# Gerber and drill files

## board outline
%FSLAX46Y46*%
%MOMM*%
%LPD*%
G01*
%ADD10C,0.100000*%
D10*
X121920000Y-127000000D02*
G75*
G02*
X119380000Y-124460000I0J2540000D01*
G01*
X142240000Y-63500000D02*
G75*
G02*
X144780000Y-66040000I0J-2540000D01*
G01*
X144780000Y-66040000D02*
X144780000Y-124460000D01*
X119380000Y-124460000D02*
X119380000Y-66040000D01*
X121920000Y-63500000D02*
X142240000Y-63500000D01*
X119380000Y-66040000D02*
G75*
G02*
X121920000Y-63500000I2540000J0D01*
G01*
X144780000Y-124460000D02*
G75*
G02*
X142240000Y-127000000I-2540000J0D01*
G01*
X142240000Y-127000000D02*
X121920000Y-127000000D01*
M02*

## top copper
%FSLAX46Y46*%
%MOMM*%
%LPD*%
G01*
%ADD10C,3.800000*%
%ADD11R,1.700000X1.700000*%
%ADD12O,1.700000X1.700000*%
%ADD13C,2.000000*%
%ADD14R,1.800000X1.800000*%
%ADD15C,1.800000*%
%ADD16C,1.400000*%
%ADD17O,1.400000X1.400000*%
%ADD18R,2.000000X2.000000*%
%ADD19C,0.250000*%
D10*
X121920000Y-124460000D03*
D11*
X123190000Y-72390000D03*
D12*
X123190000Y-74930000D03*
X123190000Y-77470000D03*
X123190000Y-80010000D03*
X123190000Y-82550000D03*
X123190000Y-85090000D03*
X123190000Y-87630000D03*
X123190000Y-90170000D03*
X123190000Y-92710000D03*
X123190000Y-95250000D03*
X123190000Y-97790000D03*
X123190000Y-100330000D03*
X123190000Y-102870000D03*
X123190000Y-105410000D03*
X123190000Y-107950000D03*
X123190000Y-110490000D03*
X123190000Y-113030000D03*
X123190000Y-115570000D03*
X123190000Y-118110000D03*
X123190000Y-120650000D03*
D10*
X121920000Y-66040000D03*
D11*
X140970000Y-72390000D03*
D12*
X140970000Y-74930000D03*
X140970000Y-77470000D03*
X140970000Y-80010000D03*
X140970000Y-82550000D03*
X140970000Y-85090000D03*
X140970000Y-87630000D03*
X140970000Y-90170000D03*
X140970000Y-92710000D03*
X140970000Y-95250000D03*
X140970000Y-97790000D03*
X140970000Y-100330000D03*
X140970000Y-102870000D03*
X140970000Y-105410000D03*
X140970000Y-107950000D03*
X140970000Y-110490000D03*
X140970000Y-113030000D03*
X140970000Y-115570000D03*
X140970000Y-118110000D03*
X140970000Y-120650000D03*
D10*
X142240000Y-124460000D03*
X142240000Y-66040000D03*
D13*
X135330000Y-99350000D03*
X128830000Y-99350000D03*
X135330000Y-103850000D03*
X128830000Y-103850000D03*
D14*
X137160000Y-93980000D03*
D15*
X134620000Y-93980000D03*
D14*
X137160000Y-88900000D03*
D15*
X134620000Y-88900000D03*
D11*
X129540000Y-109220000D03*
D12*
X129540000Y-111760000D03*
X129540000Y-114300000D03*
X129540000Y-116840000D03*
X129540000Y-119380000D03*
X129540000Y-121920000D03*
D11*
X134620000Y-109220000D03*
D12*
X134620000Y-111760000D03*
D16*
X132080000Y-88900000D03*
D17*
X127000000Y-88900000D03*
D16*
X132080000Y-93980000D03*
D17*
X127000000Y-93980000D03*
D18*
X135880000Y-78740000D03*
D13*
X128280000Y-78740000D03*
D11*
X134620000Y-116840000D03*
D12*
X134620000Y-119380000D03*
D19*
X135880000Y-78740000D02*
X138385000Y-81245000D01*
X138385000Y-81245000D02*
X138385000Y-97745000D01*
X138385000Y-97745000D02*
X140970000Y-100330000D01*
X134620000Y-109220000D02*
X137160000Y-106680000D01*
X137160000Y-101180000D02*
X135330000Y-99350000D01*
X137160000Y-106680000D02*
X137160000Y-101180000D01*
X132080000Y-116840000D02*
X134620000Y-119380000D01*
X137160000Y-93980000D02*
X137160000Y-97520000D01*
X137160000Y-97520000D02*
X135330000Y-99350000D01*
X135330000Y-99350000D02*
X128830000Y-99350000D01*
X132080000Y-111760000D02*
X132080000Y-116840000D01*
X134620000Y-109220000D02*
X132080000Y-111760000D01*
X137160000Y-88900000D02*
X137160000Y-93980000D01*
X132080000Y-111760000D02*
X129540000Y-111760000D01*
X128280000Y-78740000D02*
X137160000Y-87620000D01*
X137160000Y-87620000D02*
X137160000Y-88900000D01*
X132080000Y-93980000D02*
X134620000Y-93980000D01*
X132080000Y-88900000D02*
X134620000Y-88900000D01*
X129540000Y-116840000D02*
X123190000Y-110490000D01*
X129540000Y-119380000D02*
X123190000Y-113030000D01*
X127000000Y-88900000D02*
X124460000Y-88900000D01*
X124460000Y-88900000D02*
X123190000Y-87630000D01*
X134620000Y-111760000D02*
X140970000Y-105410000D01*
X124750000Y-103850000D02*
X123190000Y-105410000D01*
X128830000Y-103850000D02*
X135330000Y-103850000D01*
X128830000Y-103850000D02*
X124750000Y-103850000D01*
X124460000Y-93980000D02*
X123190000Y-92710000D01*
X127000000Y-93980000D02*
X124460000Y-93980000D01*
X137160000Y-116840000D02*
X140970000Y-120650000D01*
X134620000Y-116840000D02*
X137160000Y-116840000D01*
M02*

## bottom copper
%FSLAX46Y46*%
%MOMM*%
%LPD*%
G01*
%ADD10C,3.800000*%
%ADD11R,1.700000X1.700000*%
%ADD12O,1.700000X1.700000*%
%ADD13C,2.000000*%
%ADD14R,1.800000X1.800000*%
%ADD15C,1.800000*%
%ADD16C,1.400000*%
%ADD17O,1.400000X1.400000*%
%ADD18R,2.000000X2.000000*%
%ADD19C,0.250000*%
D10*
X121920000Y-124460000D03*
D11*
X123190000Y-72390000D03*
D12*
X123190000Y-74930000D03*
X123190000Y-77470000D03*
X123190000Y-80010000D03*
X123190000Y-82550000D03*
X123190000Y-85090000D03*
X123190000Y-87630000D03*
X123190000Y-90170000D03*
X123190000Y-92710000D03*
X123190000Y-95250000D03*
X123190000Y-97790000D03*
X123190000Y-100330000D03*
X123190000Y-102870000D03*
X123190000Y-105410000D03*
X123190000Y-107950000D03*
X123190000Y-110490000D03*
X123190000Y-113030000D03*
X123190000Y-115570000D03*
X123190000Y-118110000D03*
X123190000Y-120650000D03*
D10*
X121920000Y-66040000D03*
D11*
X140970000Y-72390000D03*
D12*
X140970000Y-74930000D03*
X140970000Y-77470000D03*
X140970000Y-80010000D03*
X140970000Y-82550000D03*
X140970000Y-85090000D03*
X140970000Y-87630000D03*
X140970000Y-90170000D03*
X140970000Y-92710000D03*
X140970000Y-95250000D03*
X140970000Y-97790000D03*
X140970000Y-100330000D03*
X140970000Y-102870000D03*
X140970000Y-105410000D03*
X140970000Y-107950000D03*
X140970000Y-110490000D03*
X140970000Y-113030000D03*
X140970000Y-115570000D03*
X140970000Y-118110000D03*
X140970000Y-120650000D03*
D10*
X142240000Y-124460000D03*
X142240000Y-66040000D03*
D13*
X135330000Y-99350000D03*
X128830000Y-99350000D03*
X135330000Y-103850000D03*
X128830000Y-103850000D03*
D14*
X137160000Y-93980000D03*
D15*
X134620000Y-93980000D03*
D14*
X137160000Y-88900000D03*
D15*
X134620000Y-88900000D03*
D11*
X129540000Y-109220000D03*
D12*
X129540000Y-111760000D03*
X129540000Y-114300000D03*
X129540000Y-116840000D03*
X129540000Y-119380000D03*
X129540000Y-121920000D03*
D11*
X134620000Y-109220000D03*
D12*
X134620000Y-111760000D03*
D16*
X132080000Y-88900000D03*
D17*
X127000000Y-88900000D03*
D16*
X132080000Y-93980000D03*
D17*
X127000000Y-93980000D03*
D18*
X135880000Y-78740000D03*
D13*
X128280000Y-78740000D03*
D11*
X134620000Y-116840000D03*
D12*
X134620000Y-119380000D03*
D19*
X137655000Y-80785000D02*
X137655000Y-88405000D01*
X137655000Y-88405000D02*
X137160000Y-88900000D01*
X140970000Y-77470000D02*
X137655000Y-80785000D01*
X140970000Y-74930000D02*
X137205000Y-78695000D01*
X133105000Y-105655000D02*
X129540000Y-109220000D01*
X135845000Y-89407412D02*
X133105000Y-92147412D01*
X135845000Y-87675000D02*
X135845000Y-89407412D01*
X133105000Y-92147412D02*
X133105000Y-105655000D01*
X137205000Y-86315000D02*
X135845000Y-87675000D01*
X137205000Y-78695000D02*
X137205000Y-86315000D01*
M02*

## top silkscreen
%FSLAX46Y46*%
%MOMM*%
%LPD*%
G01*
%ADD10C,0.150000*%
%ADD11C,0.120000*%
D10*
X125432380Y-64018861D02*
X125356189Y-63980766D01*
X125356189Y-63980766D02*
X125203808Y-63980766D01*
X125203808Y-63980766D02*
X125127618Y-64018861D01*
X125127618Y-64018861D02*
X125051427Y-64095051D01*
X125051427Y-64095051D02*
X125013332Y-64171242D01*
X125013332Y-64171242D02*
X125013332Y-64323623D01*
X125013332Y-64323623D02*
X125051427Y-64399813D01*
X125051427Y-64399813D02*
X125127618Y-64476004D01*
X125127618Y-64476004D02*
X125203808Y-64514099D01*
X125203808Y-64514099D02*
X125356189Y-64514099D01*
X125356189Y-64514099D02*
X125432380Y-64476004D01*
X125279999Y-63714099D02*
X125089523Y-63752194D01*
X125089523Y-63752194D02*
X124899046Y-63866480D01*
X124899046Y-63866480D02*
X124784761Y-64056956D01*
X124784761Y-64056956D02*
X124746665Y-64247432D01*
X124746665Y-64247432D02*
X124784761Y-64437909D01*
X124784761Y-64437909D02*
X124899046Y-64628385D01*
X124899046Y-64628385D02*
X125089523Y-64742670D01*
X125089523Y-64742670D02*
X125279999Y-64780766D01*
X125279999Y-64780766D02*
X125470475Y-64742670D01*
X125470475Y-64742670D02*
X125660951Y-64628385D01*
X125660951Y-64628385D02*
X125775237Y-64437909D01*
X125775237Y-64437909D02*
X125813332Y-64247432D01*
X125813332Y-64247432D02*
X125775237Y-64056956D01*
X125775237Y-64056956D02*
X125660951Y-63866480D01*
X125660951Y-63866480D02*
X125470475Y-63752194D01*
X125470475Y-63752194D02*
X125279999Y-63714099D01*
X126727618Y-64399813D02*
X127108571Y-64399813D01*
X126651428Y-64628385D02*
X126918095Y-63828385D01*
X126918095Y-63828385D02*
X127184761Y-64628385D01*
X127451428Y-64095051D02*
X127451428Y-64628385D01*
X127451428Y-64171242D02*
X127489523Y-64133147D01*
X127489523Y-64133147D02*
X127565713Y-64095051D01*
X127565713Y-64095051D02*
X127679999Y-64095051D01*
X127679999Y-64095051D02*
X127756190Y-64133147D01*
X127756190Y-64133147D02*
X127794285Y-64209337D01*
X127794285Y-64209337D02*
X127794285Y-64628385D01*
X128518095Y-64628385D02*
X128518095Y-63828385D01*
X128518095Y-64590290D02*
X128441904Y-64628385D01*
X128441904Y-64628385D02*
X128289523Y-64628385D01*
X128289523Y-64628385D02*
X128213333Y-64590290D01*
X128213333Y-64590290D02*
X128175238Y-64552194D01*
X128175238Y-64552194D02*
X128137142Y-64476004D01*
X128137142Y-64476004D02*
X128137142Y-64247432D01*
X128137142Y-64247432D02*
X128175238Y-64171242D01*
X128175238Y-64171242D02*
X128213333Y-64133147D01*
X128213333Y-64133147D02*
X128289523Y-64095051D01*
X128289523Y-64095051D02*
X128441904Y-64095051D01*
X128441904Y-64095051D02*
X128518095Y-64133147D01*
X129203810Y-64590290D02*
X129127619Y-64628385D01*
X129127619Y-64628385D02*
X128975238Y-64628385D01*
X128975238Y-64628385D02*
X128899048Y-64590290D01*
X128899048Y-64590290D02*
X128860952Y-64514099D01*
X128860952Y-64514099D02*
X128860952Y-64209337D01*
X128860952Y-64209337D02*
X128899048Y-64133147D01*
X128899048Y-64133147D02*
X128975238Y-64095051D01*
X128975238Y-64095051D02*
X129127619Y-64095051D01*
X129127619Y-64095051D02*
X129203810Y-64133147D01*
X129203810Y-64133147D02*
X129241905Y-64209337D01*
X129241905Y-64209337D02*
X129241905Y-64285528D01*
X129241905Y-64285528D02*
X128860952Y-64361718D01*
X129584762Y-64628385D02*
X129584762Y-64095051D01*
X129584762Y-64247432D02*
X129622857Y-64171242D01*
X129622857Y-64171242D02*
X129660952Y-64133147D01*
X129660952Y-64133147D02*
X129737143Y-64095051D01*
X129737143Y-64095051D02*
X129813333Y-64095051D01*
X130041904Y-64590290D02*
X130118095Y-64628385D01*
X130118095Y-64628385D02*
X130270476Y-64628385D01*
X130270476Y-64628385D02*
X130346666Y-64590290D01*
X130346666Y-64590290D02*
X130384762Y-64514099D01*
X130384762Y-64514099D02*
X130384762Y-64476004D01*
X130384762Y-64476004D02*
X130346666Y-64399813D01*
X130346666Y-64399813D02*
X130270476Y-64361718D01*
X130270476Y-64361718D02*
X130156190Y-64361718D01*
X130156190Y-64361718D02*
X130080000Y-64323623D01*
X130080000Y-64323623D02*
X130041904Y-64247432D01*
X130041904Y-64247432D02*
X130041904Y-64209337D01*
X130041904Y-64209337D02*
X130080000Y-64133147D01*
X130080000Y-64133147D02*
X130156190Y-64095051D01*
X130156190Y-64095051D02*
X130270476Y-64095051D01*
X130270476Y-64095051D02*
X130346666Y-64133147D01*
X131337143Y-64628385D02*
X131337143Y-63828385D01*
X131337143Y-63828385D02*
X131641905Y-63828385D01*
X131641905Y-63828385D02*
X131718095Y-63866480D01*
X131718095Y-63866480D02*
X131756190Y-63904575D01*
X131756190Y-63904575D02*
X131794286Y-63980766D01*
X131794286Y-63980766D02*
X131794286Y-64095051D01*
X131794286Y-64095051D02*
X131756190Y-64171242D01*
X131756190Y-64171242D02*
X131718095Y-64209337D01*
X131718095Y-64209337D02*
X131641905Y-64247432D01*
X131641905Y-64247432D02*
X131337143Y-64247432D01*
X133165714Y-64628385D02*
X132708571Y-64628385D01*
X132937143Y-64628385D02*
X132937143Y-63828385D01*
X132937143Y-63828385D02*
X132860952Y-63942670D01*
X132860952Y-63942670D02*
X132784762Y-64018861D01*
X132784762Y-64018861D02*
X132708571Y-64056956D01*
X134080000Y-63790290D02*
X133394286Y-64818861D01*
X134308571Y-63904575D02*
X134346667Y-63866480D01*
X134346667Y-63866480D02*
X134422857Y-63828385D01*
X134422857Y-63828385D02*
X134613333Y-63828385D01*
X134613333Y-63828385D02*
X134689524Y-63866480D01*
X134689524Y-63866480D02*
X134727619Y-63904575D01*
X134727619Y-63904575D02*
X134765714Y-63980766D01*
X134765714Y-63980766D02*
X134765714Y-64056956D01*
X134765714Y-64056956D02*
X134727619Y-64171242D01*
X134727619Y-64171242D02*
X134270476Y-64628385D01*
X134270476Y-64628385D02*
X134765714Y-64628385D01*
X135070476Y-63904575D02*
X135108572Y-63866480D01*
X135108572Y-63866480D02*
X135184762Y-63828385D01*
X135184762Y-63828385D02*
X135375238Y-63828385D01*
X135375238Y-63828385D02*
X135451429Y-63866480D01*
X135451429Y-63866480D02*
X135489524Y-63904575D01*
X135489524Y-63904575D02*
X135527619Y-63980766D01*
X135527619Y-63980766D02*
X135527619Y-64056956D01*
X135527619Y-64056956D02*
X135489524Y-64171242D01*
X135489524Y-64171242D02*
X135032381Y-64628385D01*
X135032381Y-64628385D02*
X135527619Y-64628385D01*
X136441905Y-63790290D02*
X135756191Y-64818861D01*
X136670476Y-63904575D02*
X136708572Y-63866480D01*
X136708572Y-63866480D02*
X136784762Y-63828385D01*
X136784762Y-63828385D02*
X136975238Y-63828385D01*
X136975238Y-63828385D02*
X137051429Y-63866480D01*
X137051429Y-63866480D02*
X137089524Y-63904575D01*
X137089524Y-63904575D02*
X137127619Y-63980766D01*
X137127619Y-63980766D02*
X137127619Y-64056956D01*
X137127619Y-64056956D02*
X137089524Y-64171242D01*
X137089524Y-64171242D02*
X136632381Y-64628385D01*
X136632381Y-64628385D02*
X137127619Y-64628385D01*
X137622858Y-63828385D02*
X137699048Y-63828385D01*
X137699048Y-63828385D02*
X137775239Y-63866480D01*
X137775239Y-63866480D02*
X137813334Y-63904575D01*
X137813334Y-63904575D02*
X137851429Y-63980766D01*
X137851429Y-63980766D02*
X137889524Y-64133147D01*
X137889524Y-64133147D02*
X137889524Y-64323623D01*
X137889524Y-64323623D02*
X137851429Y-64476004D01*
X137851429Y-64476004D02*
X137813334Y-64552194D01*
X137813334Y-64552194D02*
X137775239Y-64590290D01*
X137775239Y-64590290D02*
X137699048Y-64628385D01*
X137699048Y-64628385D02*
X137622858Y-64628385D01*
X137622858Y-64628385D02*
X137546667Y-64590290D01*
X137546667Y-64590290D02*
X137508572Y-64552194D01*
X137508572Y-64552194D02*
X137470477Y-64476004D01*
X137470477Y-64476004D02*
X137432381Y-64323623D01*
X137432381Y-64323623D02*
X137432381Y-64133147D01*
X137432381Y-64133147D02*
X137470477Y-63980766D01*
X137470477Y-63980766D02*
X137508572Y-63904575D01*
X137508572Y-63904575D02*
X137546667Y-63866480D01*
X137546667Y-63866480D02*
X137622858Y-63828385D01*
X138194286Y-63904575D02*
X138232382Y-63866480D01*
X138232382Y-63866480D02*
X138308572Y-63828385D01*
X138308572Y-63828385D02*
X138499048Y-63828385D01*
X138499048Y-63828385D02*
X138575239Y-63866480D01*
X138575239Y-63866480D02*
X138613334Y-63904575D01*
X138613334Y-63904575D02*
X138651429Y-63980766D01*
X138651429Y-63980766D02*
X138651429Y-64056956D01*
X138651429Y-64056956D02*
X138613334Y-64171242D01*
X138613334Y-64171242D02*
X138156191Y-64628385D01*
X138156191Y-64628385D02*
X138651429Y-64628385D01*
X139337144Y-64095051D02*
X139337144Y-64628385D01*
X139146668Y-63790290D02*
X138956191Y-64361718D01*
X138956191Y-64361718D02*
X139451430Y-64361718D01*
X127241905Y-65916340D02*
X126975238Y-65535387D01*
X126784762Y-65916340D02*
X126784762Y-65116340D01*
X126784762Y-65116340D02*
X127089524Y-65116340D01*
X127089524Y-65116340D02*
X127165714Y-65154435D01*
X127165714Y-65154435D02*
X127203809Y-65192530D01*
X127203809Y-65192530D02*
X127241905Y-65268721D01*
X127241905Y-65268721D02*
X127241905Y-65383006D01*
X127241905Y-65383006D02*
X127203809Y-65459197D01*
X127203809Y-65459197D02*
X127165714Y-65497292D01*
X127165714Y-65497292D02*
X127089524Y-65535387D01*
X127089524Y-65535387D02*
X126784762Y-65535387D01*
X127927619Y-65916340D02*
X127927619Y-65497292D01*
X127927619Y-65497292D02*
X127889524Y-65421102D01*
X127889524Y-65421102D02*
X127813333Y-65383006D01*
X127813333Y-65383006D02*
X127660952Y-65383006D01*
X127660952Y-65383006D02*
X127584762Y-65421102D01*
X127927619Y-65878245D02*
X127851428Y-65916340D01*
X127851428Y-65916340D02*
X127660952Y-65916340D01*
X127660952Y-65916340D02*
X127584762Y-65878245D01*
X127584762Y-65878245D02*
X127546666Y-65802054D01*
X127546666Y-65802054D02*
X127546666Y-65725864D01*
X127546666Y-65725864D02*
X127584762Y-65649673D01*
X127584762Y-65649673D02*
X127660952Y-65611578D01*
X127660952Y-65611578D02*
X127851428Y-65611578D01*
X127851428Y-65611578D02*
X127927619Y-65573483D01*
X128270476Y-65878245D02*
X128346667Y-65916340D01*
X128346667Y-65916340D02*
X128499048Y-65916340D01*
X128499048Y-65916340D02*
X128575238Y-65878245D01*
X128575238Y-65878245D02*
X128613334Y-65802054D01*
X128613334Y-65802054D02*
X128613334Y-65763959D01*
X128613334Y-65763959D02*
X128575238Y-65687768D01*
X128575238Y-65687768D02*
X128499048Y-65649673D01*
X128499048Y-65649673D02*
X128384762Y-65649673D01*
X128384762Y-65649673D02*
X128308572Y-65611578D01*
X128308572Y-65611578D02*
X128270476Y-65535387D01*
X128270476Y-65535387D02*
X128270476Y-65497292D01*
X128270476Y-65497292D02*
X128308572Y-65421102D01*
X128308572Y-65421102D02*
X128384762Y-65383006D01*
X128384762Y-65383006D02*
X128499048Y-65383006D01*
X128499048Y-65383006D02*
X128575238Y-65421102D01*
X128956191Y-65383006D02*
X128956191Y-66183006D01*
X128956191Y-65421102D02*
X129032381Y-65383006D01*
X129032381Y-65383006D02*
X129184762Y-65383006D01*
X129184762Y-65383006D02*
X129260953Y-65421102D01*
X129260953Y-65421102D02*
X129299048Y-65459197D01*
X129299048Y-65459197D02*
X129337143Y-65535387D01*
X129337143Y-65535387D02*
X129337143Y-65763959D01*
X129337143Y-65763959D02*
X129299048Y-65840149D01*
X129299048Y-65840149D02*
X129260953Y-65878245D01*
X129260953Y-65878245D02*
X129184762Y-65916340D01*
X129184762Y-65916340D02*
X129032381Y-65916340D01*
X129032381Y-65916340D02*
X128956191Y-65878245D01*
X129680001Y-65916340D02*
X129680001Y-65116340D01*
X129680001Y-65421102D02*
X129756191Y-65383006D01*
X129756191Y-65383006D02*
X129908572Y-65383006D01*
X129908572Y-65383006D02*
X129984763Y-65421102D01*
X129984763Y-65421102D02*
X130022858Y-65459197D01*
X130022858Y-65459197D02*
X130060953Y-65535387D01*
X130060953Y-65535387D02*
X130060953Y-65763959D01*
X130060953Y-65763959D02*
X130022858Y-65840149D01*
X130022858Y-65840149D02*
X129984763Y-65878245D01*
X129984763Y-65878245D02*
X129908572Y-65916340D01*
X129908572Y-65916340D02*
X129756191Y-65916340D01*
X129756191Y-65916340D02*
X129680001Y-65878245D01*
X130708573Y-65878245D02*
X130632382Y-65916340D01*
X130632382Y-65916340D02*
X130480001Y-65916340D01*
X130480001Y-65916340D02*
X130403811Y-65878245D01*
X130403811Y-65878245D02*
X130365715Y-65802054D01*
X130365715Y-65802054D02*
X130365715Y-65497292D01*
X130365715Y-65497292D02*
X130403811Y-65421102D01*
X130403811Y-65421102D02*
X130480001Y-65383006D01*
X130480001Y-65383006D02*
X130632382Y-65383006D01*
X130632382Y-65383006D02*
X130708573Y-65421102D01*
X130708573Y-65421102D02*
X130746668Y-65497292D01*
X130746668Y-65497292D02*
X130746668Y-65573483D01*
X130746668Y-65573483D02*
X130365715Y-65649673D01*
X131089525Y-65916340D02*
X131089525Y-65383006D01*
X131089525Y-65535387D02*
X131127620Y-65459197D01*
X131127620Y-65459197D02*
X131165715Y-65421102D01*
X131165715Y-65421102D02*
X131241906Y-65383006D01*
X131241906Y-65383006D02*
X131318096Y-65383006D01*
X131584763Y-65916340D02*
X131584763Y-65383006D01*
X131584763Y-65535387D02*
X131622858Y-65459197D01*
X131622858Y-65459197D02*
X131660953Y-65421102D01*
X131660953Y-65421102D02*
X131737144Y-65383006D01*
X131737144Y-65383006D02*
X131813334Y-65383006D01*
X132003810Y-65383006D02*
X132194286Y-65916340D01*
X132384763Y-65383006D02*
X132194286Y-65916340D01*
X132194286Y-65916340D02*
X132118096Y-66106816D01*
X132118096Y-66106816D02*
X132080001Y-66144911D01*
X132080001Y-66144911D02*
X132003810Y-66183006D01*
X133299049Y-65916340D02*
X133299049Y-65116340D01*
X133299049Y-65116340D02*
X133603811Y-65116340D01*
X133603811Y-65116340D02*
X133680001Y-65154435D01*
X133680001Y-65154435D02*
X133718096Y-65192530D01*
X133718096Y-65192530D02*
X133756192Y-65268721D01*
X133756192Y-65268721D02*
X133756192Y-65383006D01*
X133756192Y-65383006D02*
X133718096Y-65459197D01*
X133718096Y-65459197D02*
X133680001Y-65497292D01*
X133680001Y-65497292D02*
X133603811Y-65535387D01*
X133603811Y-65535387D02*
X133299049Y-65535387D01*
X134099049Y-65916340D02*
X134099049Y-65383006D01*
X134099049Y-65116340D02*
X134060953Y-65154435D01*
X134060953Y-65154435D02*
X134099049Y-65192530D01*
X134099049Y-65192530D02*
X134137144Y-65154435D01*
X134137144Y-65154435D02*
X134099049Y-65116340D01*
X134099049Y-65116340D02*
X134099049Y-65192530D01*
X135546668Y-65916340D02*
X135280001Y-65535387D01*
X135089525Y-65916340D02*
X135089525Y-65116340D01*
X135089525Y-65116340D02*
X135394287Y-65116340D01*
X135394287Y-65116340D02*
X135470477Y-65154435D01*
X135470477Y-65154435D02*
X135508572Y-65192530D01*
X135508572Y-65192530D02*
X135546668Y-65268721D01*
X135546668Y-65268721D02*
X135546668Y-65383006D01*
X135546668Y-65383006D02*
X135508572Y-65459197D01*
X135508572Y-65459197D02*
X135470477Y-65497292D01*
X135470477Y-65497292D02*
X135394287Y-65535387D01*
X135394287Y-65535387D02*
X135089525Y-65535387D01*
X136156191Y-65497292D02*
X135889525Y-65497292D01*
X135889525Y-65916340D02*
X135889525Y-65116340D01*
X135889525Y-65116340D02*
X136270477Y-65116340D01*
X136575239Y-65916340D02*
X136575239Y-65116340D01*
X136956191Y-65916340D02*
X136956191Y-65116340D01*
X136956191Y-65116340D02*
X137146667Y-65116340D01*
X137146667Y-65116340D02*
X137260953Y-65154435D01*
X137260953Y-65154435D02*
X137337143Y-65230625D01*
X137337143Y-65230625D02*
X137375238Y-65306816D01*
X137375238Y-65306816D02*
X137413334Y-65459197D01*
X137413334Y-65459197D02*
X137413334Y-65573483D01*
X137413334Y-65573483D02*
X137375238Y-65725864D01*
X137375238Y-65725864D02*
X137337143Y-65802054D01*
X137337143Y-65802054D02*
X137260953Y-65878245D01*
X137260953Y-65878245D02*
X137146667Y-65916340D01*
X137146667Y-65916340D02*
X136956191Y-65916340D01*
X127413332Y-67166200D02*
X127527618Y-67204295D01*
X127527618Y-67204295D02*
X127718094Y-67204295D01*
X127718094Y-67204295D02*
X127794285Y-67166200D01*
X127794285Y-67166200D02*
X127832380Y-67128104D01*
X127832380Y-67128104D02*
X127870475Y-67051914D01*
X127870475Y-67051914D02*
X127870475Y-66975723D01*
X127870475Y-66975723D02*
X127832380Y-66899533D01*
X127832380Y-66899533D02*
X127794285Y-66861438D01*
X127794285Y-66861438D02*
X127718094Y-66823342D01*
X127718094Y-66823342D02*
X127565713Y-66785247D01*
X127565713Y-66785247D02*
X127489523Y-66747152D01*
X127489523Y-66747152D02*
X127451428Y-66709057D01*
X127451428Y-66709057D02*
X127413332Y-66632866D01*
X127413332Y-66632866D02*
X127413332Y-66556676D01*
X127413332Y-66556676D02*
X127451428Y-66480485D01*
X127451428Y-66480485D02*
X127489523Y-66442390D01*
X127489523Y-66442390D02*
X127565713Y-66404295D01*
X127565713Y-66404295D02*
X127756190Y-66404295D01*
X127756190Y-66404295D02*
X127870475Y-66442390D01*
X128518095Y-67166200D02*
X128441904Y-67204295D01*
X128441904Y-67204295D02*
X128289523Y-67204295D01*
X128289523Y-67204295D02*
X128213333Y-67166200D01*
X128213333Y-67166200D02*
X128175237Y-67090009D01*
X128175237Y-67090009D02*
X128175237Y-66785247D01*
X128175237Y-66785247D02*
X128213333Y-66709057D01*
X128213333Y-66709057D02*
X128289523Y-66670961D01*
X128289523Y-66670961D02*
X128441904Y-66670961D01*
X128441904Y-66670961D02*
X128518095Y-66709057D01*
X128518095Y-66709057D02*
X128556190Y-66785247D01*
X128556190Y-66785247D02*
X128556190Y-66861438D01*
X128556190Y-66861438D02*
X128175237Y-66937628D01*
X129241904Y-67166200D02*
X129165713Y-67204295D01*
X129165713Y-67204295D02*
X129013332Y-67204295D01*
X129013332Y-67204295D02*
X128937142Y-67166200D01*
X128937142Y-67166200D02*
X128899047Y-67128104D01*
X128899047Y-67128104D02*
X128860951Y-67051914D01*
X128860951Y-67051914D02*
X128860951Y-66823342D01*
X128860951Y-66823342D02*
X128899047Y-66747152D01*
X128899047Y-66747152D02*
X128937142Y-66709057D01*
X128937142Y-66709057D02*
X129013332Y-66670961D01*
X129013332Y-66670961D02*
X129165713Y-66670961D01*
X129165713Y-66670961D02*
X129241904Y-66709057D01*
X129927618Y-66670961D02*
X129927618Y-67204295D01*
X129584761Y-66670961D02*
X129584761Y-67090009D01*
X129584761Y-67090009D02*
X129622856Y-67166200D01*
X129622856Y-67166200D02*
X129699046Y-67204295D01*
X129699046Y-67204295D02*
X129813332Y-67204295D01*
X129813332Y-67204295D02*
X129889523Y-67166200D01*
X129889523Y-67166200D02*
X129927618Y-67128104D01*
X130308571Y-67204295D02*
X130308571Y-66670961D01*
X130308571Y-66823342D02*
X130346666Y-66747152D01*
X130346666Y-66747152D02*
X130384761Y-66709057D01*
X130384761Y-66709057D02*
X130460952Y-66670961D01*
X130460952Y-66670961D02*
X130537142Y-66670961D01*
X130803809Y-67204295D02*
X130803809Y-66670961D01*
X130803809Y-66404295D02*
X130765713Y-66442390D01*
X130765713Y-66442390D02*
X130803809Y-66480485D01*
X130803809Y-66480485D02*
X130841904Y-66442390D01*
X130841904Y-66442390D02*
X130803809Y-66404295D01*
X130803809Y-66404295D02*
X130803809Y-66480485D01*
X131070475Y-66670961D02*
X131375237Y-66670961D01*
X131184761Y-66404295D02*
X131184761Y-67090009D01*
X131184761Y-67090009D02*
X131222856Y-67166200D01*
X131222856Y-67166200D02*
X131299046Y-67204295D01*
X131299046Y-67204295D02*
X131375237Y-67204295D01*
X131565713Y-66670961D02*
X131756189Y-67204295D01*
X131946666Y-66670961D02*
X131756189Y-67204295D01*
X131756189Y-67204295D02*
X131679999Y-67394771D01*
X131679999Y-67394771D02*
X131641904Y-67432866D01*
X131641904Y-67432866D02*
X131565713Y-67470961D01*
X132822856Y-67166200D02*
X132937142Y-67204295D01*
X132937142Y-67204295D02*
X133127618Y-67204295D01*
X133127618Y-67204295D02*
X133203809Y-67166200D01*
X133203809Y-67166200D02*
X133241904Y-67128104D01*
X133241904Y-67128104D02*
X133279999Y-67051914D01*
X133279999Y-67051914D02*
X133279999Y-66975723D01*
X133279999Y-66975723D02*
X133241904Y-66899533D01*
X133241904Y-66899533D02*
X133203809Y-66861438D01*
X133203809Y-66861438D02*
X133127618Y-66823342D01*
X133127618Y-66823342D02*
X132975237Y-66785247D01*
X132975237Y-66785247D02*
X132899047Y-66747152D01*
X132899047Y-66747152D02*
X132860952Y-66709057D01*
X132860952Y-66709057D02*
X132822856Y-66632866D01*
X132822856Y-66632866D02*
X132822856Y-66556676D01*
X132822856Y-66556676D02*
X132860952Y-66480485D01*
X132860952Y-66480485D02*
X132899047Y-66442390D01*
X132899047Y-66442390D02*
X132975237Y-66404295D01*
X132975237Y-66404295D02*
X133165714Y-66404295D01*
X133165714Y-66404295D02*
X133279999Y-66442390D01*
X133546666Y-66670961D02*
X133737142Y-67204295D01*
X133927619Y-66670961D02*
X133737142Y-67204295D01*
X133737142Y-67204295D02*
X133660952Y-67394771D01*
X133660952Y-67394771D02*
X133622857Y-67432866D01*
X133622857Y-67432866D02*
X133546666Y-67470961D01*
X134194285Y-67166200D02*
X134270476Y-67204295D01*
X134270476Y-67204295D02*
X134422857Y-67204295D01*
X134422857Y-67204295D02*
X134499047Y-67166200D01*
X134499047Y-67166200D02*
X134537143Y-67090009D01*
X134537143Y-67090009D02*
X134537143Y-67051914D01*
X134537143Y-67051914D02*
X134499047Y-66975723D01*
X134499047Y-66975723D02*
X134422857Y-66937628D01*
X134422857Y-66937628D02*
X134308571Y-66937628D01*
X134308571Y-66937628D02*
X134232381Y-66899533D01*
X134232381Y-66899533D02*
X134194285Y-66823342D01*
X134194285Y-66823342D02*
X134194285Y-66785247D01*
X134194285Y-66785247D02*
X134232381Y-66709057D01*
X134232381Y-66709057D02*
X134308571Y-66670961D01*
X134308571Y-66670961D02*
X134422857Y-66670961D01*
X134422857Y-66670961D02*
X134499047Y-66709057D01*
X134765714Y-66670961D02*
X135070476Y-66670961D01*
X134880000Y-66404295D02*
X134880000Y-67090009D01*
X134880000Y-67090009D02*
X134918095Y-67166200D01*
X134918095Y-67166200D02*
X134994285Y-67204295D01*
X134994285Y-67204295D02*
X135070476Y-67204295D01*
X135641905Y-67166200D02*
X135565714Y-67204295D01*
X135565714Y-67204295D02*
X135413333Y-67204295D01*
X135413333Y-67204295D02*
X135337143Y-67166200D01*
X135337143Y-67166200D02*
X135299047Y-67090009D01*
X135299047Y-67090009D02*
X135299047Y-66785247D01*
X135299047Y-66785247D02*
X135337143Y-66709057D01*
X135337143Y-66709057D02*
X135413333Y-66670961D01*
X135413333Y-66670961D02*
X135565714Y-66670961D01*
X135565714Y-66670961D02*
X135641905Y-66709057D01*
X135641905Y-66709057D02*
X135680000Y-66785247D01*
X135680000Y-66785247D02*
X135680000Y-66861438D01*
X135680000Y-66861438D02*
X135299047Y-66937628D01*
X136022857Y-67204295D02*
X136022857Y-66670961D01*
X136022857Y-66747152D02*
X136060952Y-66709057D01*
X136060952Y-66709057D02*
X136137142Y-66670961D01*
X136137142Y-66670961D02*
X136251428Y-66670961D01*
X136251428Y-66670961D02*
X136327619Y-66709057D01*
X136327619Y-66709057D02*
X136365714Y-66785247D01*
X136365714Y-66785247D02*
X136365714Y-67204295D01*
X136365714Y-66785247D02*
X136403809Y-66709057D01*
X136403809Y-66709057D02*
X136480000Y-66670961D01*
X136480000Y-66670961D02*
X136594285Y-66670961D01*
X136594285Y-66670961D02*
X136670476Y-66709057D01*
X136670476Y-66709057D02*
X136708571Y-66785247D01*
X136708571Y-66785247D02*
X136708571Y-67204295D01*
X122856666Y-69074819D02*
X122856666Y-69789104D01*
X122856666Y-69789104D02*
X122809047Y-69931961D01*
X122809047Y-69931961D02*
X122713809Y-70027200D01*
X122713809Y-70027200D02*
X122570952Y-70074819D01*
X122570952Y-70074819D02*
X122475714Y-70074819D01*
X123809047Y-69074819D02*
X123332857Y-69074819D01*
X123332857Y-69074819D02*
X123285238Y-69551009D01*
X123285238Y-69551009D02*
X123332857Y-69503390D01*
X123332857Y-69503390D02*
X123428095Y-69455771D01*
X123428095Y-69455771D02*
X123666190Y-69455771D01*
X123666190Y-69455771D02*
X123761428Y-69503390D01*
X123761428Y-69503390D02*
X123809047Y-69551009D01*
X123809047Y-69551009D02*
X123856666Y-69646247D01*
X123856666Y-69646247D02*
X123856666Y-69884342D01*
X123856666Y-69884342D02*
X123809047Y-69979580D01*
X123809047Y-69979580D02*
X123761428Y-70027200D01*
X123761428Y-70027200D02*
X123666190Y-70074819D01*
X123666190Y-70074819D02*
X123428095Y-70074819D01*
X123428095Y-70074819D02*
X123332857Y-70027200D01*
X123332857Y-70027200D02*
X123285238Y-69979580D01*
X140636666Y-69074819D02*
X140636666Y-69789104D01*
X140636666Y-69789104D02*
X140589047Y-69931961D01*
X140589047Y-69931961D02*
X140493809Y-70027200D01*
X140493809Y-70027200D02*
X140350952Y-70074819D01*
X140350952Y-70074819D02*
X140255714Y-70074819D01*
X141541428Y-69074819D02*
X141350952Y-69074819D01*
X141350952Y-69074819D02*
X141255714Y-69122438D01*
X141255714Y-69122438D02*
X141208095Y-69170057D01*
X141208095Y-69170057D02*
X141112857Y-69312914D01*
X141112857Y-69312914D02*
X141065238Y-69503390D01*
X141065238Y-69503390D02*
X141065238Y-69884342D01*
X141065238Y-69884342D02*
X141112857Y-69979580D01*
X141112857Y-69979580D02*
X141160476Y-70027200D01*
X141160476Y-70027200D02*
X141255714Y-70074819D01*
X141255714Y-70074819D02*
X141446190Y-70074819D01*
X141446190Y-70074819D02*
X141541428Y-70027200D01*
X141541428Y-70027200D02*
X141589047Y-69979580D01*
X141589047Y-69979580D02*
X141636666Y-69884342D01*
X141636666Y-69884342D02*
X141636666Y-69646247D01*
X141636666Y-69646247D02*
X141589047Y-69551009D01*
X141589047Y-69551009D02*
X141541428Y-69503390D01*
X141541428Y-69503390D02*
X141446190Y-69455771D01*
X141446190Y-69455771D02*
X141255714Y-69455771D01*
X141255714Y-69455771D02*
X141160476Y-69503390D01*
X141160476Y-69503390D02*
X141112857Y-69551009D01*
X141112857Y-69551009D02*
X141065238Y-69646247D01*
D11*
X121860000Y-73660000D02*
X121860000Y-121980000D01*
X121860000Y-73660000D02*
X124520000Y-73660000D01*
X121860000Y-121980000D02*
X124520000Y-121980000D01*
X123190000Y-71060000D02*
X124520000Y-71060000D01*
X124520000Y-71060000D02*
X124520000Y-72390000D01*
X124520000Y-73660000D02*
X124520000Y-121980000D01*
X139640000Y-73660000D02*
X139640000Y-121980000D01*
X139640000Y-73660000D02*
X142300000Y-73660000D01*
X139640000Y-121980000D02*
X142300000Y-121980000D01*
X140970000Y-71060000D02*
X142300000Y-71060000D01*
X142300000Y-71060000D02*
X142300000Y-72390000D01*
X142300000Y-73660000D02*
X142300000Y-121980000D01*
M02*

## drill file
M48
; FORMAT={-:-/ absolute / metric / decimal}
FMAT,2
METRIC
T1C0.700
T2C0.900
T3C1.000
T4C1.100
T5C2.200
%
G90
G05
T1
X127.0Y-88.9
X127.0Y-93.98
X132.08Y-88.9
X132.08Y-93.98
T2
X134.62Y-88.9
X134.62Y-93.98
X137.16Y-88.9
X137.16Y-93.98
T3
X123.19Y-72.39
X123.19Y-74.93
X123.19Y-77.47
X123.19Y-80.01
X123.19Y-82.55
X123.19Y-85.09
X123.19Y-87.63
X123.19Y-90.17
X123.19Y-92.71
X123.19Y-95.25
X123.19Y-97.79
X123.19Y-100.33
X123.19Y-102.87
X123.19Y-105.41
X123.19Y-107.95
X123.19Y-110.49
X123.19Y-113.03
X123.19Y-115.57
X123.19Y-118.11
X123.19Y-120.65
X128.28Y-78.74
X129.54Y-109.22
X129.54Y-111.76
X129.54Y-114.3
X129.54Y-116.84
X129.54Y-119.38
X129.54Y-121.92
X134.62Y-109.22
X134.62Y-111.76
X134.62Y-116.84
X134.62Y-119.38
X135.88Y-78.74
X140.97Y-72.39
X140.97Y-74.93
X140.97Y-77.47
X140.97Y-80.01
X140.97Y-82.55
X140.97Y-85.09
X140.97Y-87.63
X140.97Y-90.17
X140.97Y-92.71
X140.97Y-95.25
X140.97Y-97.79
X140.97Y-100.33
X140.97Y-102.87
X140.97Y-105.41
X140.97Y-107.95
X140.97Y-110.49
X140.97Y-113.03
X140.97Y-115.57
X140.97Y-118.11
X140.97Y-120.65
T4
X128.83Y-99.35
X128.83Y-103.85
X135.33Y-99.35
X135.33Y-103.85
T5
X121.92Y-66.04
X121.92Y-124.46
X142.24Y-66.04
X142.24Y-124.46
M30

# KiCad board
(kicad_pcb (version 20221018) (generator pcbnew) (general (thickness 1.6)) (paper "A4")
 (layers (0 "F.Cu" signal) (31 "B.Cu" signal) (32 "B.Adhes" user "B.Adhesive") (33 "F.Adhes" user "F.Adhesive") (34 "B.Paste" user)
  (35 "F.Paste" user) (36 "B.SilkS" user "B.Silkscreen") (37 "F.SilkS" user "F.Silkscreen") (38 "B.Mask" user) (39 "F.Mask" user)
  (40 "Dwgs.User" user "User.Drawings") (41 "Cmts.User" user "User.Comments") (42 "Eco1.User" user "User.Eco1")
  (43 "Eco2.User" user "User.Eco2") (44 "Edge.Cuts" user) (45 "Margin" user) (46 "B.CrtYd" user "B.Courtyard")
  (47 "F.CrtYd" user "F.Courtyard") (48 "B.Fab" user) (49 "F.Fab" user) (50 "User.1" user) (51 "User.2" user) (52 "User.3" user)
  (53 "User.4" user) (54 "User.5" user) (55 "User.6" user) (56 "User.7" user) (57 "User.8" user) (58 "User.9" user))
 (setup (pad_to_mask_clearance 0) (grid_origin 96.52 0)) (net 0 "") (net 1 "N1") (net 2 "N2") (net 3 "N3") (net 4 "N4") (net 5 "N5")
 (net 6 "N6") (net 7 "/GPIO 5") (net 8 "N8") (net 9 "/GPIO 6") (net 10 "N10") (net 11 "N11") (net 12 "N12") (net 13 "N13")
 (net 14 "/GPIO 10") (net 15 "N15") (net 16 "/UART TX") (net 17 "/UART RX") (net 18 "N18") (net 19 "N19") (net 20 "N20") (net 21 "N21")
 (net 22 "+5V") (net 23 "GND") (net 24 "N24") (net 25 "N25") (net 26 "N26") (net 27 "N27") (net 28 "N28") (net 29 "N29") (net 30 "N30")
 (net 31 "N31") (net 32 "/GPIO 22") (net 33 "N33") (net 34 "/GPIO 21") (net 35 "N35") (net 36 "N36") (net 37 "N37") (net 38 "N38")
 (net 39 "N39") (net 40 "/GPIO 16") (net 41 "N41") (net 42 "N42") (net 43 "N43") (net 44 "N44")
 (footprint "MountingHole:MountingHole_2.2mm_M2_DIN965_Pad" (layer "F.Cu") (at 121.92 124.46)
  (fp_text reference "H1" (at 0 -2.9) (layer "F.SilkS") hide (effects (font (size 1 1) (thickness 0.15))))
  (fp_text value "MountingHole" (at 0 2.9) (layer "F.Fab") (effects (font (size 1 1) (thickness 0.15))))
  (pad "1" thru_hole circle (at 0 0) (size 3.8 3.8) (drill 2.2) (layers "*.Cu" "*.Mask")))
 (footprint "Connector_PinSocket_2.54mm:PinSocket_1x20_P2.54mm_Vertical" (layer "F.Cu") (at 123.19 72.39)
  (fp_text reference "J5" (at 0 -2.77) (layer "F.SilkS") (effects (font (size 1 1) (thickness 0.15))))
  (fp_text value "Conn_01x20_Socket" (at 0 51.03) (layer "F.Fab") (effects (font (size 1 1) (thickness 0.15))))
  (fp_line (start -1.33 1.27) (end -1.33 49.59) (stroke (width 0.12) (type solid)) (layer "F.SilkS"))
  (fp_line (start -1.33 1.27) (end 1.33 1.27) (stroke (width 0.12) (type solid)) (layer "F.SilkS"))
  (fp_line (start -1.33 49.59) (end 1.33 49.59) (stroke (width 0.12) (type solid)) (layer "F.SilkS"))
  (fp_line (start 0 -1.33) (end 1.33 -1.33) (stroke (width 0.12) (type solid)) (layer "F.SilkS"))
  (fp_line (start 1.33 -1.33) (end 1.33 0) (stroke (width 0.12) (type solid)) (layer "F.SilkS"))
  (fp_line (start 1.33 1.27) (end 1.33 49.59) (stroke (width 0.12) (type solid)) (layer "F.SilkS"))
  (pad "1" thru_hole rect (at 0 0) (size 1.7 1.7) (drill 1) (layers "*.Cu" "*.Mask") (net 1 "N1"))
  (pad "2" thru_hole oval (at 0 2.54) (size 1.7 1.7) (drill 1) (layers "*.Cu" "*.Mask") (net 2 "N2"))
  (pad "3" thru_hole oval (at 0 5.08) (size 1.7 1.7) (drill 1) (layers "*.Cu" "*.Mask") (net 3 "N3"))
  (pad "4" thru_hole oval (at 0 7.62) (size 1.7 1.7) (drill 1) (layers "*.Cu" "*.Mask") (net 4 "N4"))
  (pad "5" thru_hole oval (at 0 10.16) (size 1.7 1.7) (drill 1) (layers "*.Cu" "*.Mask") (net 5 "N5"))
  (pad "6" thru_hole oval (at 0 12.7) (size 1.7 1.7) (drill 1) (layers "*.Cu" "*.Mask") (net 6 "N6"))
  (pad "7" thru_hole oval (at 0 15.24) (size 1.7 1.7) (drill 1) (layers "*.Cu" "*.Mask") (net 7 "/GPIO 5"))
  (pad "8" thru_hole oval (at 0 17.78) (size 1.7 1.7) (drill 1) (layers "*.Cu" "*.Mask") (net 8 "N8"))
  (pad "9" thru_hole oval (at 0 20.32) (size 1.7 1.7) (drill 1) (layers "*.Cu" "*.Mask") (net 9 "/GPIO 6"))
  (pad "10" thru_hole oval (at 0 22.86) (size 1.7 1.7) (drill 1) (layers "*.Cu" "*.Mask") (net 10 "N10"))
  (pad "11" thru_hole oval (at 0 25.4) (size 1.7 1.7) (drill 1) (layers "*.Cu" "*.Mask") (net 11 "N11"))
  (pad "12" thru_hole oval (at 0 27.94) (size 1.7 1.7) (drill 1) (layers "*.Cu" "*.Mask") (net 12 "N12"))
  (pad "13" thru_hole oval (at 0 30.48) (size 1.7 1.7) (drill 1) (layers "*.Cu" "*.Mask") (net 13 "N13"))
  (pad "14" thru_hole oval (at 0 33.02) (size 1.7 1.7) (drill 1) (layers "*.Cu" "*.Mask") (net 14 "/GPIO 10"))
  (pad "15" thru_hole oval (at 0 35.56) (size 1.7 1.7) (drill 1) (layers "*.Cu" "*.Mask") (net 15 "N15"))
  (pad "16" thru_hole oval (at 0 38.1) (size 1.7 1.7) (drill 1) (layers "*.Cu" "*.Mask") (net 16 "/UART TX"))
  (pad "17" thru_hole oval (at 0 40.64) (size 1.7 1.7) (drill 1) (layers "*.Cu" "*.Mask") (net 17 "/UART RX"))
  (pad "18" thru_hole oval (at 0 43.18) (size 1.7 1.7) (drill 1) (layers "*.Cu" "*.Mask") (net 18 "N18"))
  (pad "19" thru_hole oval (at 0 45.72) (size 1.7 1.7) (drill 1) (layers "*.Cu" "*.Mask") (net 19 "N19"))
  (pad "20" thru_hole oval (at 0 48.26) (size 1.7 1.7) (drill 1) (layers "*.Cu" "*.Mask") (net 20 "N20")))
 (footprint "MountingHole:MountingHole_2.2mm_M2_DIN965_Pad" (layer "F.Cu") (at 121.92 66.04)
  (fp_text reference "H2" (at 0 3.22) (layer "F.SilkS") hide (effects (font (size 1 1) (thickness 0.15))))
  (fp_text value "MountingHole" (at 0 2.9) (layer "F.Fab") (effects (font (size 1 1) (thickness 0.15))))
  (pad "1" thru_hole circle (at 0 0) (size 3.8 3.8) (drill 2.2) (layers "*.Cu" "*.Mask")))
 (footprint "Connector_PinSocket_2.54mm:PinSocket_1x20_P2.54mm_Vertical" (layer "F.Cu") (at 140.97 72.39)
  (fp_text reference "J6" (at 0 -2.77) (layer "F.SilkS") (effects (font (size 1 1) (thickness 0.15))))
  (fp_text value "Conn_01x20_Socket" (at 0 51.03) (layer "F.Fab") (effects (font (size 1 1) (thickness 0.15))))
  (fp_line (start -1.33 1.27) (end -1.33 49.59) (stroke (width 0.12) (type solid)) (layer "F.SilkS"))
  (fp_line (start -1.33 1.27) (end 1.33 1.27) (stroke (width 0.12) (type solid)) (layer "F.SilkS"))
  (fp_line (start -1.33 49.59) (end 1.33 49.59) (stroke (width 0.12) (type solid)) (layer "F.SilkS"))
  (fp_line (start 0 -1.33) (end 1.33 -1.33) (stroke (width 0.12) (type solid)) (layer "F.SilkS"))
  (fp_line (start 1.33 -1.33) (end 1.33 0) (stroke (width 0.12) (type solid)) (layer "F.SilkS"))
  (fp_line (start 1.33 1.27) (end 1.33 49.59) (stroke (width 0.12) (type solid)) (layer "F.SilkS"))
  (pad "1" thru_hole rect (at 0 0) (size 1.7 1.7) (drill 1) (layers "*.Cu" "*.Mask") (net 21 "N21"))
  (pad "2" thru_hole oval (at 0 2.54) (size 1.7 1.7) (drill 1) (layers "*.Cu" "*.Mask") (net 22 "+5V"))
  (pad "3" thru_hole oval (at 0 5.08) (size 1.7 1.7) (drill 1) (layers "*.Cu" "*.Mask") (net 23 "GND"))
  (pad "4" thru_hole oval (at 0 7.62) (size 1.7 1.7) (drill 1) (layers "*.Cu" "*.Mask") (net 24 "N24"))
  (pad "5" thru_hole oval (at 0 10.16) (size 1.7 1.7) (drill 1) (layers "*.Cu" "*.Mask") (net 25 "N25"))
  (pad "6" thru_hole oval (at 0 12.7) (size 1.7 1.7) (drill 1) (layers "*.Cu" "*.Mask") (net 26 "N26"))
  (pad "7" thru_hole oval (at 0 15.24) (size 1.7 1.7) (drill 1) (layers "*.Cu" "*.Mask") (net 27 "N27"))
  (pad "8" thru_hole oval (at 0 17.78) (size 1.7 1.7) (drill 1) (layers "*.Cu" "*.Mask") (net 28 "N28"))
  (pad "9" thru_hole oval (at 0 20.32) (size 1.7 1.7) (drill 1) (layers "*.Cu" "*.Mask") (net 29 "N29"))
  (pad "10" thru_hole oval (at 0 22.86) (size 1.7 1.7) (drill 1) (layers "*.Cu" "*.Mask") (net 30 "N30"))
  (pad "11" thru_hole oval (at 0 25.4) (size 1.7 1.7) (drill 1) (layers "*.Cu" "*.Mask") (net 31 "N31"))
  (pad "12" thru_hole oval (at 0 27.94) (size 1.7 1.7) (drill 1) (layers "*.Cu" "*.Mask") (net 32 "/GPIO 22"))
  (pad "13" thru_hole oval (at 0 30.48) (size 1.7 1.7) (drill 1) (layers "*.Cu" "*.Mask") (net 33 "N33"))
  (pad "14" thru_hole oval (at 0 33.02) (size 1.7 1.7) (drill 1) (layers "*.Cu" "*.Mask") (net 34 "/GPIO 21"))
  (pad "15" thru_hole oval (at 0 35.56) (size 1.7 1.7) (drill 1) (layers "*.Cu" "*.Mask") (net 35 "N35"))
  (pad "16" thru_hole oval (at 0 38.1) (size 1.7 1.7) (drill 1) (layers "*.Cu" "*.Mask") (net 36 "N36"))
  (pad "17" thru_hole oval (at 0 40.64) (size 1.7 1.7) (drill 1) (layers "*.Cu" "*.Mask") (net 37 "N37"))
  (pad "18" thru_hole oval (at 0 43.18) (size 1.7 1.7) (drill 1) (layers "*.Cu" "*.Mask") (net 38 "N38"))
  (pad "19" thru_hole oval (at 0 45.72) (size 1.7 1.7) (drill 1) (layers "*.Cu" "*.Mask") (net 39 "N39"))
  (pad "20" thru_hole oval (at 0 48.26) (size 1.7 1.7) (drill 1) (layers "*.Cu" "*.Mask") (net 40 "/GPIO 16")))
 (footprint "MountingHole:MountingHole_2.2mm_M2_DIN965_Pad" (layer "F.Cu") (at 142.24 124.46)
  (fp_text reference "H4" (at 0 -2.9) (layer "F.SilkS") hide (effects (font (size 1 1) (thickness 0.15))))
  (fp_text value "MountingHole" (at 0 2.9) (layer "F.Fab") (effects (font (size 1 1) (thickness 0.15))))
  (pad "1" thru_hole circle (at 0 0) (size 3.8 3.8) (drill 2.2) (layers "*.Cu" "*.Mask")))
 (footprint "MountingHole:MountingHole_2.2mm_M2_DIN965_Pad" (layer "F.Cu") (at 142.24 66.04)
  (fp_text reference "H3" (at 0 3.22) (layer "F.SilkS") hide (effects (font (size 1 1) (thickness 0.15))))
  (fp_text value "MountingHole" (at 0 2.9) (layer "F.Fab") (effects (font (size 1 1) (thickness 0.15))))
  (pad "1" thru_hole circle (at 0 0) (size 3.8 3.8) (drill 2.2) (layers "*.Cu" "*.Mask")))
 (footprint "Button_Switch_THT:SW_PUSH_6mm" (layer "B.Cu") (at 135.33 99.35 180)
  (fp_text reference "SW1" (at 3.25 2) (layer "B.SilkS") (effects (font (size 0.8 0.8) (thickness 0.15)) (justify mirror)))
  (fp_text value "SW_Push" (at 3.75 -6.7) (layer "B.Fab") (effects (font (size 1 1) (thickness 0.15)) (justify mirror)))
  (pad "1" thru_hole circle (at 0 0 90) (size 2 2) (drill 1.1) (layers "*.Cu" "*.Mask") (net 23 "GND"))
  (pad "1" thru_hole circle (at 6.5 0 90) (size 2 2) (drill 1.1) (layers "*.Cu" "*.Mask") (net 23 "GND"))
  (pad "2" thru_hole circle (at 0 -4.5 90) (size 2 2) (drill 1.1) (layers "*.Cu" "*.Mask") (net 14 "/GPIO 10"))
  (pad "2" thru_hole circle (at 6.5 -4.5 90) (size 2 2) (drill 1.1) (layers "*.Cu" "*.Mask") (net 14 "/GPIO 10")))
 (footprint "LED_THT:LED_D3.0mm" (layer "B.Cu") (at 137.16 93.98 180)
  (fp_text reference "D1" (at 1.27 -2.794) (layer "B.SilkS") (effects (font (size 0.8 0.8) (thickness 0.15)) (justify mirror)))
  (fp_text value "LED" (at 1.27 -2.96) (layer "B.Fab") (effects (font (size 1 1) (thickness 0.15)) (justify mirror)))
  (pad "1" thru_hole rect (at 0 0 180) (size 1.8 1.8) (drill 0.9) (layers "*.Cu" "*.Mask") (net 23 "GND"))
  (pad "2" thru_hole circle (at 2.54 0 180) (size 1.8 1.8) (drill 0.9) (layers "*.Cu" "*.Mask") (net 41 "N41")))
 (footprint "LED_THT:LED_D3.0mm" (layer "B.Cu") (at 137.16 88.9 180)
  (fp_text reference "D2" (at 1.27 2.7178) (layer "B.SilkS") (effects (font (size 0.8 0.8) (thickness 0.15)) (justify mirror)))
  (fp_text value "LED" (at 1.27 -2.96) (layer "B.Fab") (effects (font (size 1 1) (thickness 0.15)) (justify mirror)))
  (pad "1" thru_hole rect (at 0 0 180) (size 1.8 1.8) (drill 0.9) (layers "*.Cu" "*.Mask") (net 23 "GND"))
  (pad "2" thru_hole circle (at 2.54 0 180) (size 1.8 1.8) (drill 0.9) (layers "*.Cu" "*.Mask") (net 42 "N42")))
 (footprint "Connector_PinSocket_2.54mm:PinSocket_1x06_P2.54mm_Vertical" (layer "B.Cu") (at 129.54 109.22 180)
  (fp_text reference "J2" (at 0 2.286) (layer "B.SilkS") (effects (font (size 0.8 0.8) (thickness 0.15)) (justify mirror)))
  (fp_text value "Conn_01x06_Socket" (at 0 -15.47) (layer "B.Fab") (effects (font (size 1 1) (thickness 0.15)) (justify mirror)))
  (pad "1" thru_hole rect (at 0 0 180) (size 1.7 1.7) (drill 1) (layers "*.Cu" "*.Mask") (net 22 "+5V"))
  (pad "2" thru_hole oval (at 0 -2.54 180) (size 1.7 1.7) (drill 1) (layers "*.Cu" "*.Mask") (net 23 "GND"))
  (pad "3" thru_hole oval (at 0 -5.08 180) (size 1.7 1.7) (drill 1) (layers "*.Cu" "*.Mask") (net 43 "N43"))
  (pad "4" thru_hole oval (at 0 -7.62 180) (size 1.7 1.7) (drill 1) (layers "*.Cu" "*.Mask") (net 16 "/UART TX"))
  (pad "5" thru_hole oval (at 0 -10.16 180) (size 1.7 1.7) (drill 1) (layers "*.Cu" "*.Mask") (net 17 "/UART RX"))
  (pad "6" thru_hole oval (at 0 -12.7 180) (size 1.7 1.7) (drill 1) (layers "*.Cu" "*.Mask") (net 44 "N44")))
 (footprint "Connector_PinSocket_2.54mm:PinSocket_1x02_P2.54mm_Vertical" (layer "B.Cu") (at 134.62 109.22 180)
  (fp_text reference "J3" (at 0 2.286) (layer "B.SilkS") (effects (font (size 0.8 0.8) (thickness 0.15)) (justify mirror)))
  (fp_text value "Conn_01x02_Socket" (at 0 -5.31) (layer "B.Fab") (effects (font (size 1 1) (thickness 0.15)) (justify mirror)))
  (pad "1" thru_hole rect (at 0 0 180) (size 1.7 1.7) (drill 1) (layers "*.Cu" "*.Mask") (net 23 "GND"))
  (pad "2" thru_hole oval (at 0 -2.54 180) (size 1.7 1.7) (drill 1) (layers "*.Cu" "*.Mask") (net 34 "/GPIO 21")))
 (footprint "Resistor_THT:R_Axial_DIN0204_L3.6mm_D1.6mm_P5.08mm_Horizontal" (layer "B.Cu") (at 132.08 88.9 180)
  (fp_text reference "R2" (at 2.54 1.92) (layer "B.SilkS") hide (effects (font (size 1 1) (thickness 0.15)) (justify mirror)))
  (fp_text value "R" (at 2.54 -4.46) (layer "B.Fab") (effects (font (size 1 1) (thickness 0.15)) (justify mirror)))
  (pad "1" thru_hole circle (at 0 0 180) (size 1.4 1.4) (drill 0.7) (layers "*.Cu" "*.Mask") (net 42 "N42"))
  (pad "2" thru_hole oval (at 5.08 0 180) (size 1.4 1.4) (drill 0.7) (layers "*.Cu" "*.Mask") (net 7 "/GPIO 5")))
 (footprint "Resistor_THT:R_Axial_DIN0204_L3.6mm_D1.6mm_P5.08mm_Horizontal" (layer "B.Cu") (at 132.08 93.98 180)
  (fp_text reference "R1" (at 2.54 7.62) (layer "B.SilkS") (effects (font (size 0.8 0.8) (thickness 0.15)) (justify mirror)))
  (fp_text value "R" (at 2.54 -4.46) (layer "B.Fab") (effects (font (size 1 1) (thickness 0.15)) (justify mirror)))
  (pad "1" thru_hole circle (at 0 0 180) (size 1.4 1.4) (drill 0.7) (layers "*.Cu" "*.Mask") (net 41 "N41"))
  (pad "2" thru_hole oval (at 5.08 0 180) (size 1.4 1.4) (drill 0.7) (layers "*.Cu" "*.Mask") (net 9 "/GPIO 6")))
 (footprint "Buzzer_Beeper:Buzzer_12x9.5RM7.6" (layer "B.Cu") (at 135.88 78.74 180)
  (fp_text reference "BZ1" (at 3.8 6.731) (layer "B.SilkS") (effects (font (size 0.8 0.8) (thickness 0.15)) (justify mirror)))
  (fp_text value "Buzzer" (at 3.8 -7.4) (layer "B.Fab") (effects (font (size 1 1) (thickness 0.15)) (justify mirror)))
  (pad "1" thru_hole rect (at 0 0 180) (size 2 2) (drill 1) (layers "*.Cu" "*.Mask") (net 32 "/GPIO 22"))
  (pad "2" thru_hole circle (at 7.6 0 180) (size 2 2) (drill 1) (layers "*.Cu" "*.Mask") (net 23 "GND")))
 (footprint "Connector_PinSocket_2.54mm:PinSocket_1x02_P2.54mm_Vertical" (layer "B.Cu") (at 134.62 116.84 180)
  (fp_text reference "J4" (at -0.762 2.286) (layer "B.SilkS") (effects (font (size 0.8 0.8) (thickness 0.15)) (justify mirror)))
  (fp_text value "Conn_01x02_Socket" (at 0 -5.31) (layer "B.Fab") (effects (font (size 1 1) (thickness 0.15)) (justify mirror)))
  (pad "1" thru_hole rect (at 0 0 180) (size 1.7 1.7) (drill 1) (layers "*.Cu" "*.Mask") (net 40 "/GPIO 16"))
  (pad "2" thru_hole oval (at 0 -2.54 180) (size 1.7 1.7) (drill 1) (layers "*.Cu" "*.Mask") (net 23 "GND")))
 (gr_arc (start 121.92 127) (mid 120.123949 126.256051) (end 119.38 124.46) (stroke (width 0.1) (type default)) (layer "Edge.Cuts"))
 (gr_arc (start 142.24 63.5) (mid 144.036051 64.243949) (end 144.78 66.04) (stroke (width 0.1) (type default)) (layer "Edge.Cuts"))
 (gr_line (start 144.78 66.04) (end 144.78 124.46) (stroke (width 0.1) (type default)) (layer "Edge.Cuts"))
 (gr_line (start 119.38 124.46) (end 119.38 66.04) (stroke (width 0.1) (type default)) (layer "Edge.Cuts"))
 (gr_line (start 121.92 63.5) (end 142.24 63.5) (stroke (width 0.1) (type default)) (layer "Edge.Cuts"))
 (gr_arc (start 119.38 66.04) (mid 120.123949 64.243949) (end 121.92 63.5) (stroke (width 0.1) (type default)) (layer "Edge.Cuts"))
 (gr_arc (start 144.78 124.46) (mid 144.036051 126.256051) (end 142.24 127) (stroke (width 0.1) (type default)) (layer "Edge.Cuts"))
 (gr_line (start 142.24 127) (end 121.92 127) (stroke (width 0.1) (type default)) (layer "Edge.Cuts"))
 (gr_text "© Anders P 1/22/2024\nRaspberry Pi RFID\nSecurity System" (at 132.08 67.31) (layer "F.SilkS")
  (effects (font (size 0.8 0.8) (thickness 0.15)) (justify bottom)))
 (segment (start 135.88 78.74) (end 138.385 81.245) (width 0.25) (layer "F.Cu") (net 32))
 (segment (start 138.385 81.245) (end 138.385 97.745) (width 0.25) (layer "F.Cu") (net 32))
 (segment (start 138.385 97.745) (end 140.97 100.33) (width 0.25) (layer "F.Cu") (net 32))
 (segment (start 134.62 109.22) (end 137.16 106.68) (width 0.25) (layer "F.Cu") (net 23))
 (segment (start 137.16 101.18) (end 135.33 99.35) (width 0.25) (layer "F.Cu") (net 23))
 (segment (start 137.16 106.68) (end 137.16 101.18) (width 0.25) (layer "F.Cu") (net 23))
 (segment (start 132.08 116.84) (end 134.62 119.38) (width 0.25) (layer "F.Cu") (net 23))
 (segment (start 137.16 93.98) (end 137.16 97.52) (width 0.25) (layer "F.Cu") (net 23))
 (segment (start 137.16 97.52) (end 135.33 99.35) (width 0.25) (layer "F.Cu") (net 23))
 (segment (start 135.33 99.35) (end 128.83 99.35) (width 0.25) (layer "F.Cu") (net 23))
 (segment (start 132.08 111.76) (end 132.08 116.84) (width 0.25) (layer "F.Cu") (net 23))
 (segment (start 134.62 109.22) (end 132.08 111.76) (width 0.25) (layer "F.Cu") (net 23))
 (segment (start 137.16 88.9) (end 137.16 93.98) (width 0.25) (layer "F.Cu") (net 23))
 (segment (start 132.08 111.76) (end 129.54 111.76) (width 0.25) (layer "F.Cu") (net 23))
 (segment (start 128.28 78.74) (end 137.16 87.62) (width 0.25) (layer "F.Cu") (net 23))
 (segment (start 137.16 87.62) (end 137.16 88.9) (width 0.25) (layer "F.Cu") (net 23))
 (segment (start 137.655 80.785) (end 137.655 88.405) (width 0.25) (layer "B.Cu") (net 23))
 (segment (start 137.655 88.405) (end 137.16 88.9) (width 0.25) (layer "B.Cu") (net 23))
 (segment (start 140.97 77.47) (end 137.655 80.785) (width 0.25) (layer "B.Cu") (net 23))
 (segment (start 132.08 93.98) (end 134.62 93.98) (width 0.25) (layer "F.Cu") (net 41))
 (segment (start 132.08 88.9) (end 134.62 88.9) (width 0.25) (layer "F.Cu") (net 42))
 (segment (start 140.97 74.93) (end 137.205 78.695) (width 0.25) (layer "B.Cu") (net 22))
 (segment (start 133.105 105.655) (end 129.54 109.22) (width 0.25) (layer "B.Cu") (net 22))
 (segment (start 135.845 89.407412) (end 133.105 92.147412) (width 0.25) (layer "B.Cu") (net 22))
 (segment (start 135.845 87.675) (end 135.845 89.407412) (width 0.25) (layer "B.Cu") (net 22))
 (segment (start 133.105 92.147412) (end 133.105 105.655) (width 0.25) (layer "B.Cu") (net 22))
 (segment (start 137.205 86.315) (end 135.845 87.675) (width 0.25) (layer "B.Cu") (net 22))
 (segment (start 137.205 78.695) (end 137.205 86.315) (width 0.25) (layer "B.Cu") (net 22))
 (segment (start 129.54 116.84) (end 123.19 110.49) (width 0.25) (layer "F.Cu") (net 16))
 (segment (start 129.54 119.38) (end 123.19 113.03) (width 0.25) (layer "F.Cu") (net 17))
 (segment (start 127 88.9) (end 124.46 88.9) (width 0.25) (layer "F.Cu") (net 7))
 (segment (start 124.46 88.9) (end 123.19 87.63) (width 0.25) (layer "F.Cu") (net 7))
 (segment (start 134.62 111.76) (end 140.97 105.41) (width 0.25) (layer "F.Cu") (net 34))
 (segment (start 124.75 103.85) (end 123.19 105.41) (width 0.25) (layer "F.Cu") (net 14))
 (segment (start 128.83 103.85) (end 135.33 103.85) (width 0.25) (layer "F.Cu") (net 14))
 (segment (start 128.83 103.85) (end 124.75 103.85) (width 0.25) (layer "F.Cu") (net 14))
 (segment (start 124.46 93.98) (end 123.19 92.71) (width 0.25) (layer "F.Cu") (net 9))
 (segment (start 127 93.98) (end 124.46 93.98) (width 0.25) (layer "F.Cu") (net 9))
 (segment (start 137.16 116.84) (end 140.97 120.65) (width 0.25) (layer "F.Cu") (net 40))
 (segment (start 134.62 116.84) (end 137.16 116.84) (width 0.25) (layer "F.Cu") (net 40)))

